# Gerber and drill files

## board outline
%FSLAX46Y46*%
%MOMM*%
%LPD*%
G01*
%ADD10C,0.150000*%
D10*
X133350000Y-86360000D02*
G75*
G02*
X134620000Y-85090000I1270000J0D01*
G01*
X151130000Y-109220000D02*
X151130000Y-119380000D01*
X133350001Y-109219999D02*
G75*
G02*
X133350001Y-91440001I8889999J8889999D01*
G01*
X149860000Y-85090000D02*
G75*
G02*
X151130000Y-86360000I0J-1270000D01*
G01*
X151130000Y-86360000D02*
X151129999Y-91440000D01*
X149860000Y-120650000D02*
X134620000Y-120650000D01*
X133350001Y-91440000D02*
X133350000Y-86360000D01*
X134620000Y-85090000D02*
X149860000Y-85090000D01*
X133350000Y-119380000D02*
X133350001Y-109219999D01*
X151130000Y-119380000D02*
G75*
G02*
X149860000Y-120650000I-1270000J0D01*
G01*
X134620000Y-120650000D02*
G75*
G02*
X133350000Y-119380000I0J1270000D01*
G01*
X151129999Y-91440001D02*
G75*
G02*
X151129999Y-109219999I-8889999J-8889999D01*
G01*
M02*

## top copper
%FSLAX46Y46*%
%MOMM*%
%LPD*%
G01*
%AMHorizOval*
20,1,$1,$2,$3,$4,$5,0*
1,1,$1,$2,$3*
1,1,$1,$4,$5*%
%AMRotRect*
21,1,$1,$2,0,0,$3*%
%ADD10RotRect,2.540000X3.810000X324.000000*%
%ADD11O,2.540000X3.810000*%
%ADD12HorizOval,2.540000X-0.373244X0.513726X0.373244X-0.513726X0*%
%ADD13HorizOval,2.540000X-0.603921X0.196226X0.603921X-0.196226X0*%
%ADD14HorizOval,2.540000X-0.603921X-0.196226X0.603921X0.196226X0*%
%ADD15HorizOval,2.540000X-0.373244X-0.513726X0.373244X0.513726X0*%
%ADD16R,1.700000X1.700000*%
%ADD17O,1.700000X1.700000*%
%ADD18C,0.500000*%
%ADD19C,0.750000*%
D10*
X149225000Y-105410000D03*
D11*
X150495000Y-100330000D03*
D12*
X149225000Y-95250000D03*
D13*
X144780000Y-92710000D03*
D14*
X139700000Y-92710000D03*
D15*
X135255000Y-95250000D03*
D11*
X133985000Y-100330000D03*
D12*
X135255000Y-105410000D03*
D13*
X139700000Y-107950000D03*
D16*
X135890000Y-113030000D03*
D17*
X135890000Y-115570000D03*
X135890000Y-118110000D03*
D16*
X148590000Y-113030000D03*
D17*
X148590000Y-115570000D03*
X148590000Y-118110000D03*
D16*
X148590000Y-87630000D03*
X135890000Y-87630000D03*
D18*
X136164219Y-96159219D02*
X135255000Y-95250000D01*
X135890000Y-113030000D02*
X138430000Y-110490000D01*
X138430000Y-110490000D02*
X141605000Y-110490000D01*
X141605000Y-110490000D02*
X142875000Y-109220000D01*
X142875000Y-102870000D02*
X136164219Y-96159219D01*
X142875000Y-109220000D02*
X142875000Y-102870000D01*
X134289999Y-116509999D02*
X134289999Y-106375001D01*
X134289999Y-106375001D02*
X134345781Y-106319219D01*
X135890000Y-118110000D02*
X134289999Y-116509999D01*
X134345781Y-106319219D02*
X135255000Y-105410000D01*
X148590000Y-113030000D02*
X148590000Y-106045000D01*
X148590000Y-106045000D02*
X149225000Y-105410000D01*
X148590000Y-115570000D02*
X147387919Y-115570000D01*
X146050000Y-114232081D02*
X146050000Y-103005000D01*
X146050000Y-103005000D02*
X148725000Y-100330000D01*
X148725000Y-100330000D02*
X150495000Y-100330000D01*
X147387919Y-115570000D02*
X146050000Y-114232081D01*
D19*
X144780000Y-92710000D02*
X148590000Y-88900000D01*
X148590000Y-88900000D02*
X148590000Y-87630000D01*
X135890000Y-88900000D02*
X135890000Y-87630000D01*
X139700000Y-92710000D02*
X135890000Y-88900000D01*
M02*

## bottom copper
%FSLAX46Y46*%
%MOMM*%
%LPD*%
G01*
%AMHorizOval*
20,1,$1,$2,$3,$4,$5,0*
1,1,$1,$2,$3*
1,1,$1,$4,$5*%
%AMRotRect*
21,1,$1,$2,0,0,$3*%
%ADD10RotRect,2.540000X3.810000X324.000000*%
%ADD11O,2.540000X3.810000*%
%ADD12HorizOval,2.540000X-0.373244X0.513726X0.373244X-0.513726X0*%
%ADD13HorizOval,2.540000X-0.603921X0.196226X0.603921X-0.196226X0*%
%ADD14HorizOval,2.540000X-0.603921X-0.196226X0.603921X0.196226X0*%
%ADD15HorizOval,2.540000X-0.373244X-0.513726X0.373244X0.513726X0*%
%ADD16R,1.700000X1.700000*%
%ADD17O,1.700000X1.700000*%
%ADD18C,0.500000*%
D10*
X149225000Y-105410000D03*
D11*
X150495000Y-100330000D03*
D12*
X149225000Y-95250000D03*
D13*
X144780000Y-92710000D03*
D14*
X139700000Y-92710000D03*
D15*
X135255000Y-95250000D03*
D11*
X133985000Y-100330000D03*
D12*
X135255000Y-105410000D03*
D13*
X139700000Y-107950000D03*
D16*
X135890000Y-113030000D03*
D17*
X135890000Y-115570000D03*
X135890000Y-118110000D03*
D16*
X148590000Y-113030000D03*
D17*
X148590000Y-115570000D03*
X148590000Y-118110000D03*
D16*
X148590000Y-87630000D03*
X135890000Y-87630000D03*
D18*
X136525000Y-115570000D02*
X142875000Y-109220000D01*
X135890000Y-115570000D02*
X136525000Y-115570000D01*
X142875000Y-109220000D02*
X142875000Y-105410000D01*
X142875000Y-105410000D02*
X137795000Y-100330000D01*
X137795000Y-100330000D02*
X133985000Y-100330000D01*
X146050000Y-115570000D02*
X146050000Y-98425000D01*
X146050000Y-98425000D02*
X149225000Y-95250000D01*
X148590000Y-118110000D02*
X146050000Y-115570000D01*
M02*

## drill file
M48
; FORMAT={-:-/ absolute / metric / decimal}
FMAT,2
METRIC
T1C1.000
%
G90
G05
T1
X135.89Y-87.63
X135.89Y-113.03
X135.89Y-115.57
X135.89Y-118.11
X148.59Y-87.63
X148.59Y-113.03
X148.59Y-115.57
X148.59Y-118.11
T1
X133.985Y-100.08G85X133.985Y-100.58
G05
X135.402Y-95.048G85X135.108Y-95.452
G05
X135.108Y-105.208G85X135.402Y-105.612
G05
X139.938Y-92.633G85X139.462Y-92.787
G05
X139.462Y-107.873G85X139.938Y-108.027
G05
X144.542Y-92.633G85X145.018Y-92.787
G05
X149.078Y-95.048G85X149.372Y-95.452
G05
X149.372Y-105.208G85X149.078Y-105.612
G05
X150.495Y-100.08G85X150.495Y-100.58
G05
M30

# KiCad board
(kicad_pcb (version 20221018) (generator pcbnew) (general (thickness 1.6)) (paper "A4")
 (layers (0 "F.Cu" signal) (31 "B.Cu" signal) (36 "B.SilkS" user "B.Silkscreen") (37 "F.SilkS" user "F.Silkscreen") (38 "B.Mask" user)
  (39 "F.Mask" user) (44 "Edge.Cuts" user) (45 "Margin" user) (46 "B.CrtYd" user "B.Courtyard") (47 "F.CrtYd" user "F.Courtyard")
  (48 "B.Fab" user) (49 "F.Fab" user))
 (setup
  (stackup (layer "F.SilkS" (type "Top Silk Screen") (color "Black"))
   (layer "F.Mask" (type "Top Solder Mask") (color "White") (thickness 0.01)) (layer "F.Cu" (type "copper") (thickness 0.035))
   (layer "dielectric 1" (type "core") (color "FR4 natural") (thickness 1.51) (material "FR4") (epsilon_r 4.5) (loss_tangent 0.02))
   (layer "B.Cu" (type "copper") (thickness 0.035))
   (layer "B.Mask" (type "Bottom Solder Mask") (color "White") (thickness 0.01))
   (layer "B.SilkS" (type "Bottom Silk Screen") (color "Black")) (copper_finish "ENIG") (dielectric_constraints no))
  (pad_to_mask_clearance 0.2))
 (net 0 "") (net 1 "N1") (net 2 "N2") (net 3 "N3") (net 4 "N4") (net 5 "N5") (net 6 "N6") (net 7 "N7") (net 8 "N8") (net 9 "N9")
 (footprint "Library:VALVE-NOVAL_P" (layer "F.Cu") (at 149.86 105.41)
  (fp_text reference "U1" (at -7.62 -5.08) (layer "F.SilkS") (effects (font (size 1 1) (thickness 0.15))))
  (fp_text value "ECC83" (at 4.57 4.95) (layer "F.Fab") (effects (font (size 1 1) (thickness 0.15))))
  (pad "1" thru_hole rect (at -0.635 0 324) (size 2.54 3.81) (drill oval 1 1.5) (layers "*.Cu" "*.Mask") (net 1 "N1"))
  (pad "2" thru_hole oval (at 0.635 -5.08) (size 2.54 3.81) (drill oval 1 1.5) (layers "*.Cu" "*.Mask") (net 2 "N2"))
  (pad "3" thru_hole oval (at -0.635 -10.16 36) (size 2.54 3.81) (drill oval 1 1.5) (layers "*.Cu" "*.Mask") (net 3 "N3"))
  (pad "4" thru_hole oval (at -5.08 -12.7 72) (size 2.54 3.81) (drill oval 1 1.5) (layers "*.Cu" "*.Mask") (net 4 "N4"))
  (pad "5" thru_hole oval (at -10.16 -12.7 288) (size 2.54 3.81) (drill oval 1 1.5) (layers "*.Cu" "*.Mask") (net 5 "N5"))
  (pad "6" thru_hole oval (at -14.605 -10.16 324) (size 2.54 3.81) (drill oval 1 1.5) (layers "*.Cu" "*.Mask") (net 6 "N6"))
  (pad "7" thru_hole oval (at -15.875 -5.08) (size 2.54 3.81) (drill oval 1 1.5) (layers "*.Cu" "*.Mask") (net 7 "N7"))
  (pad "8" thru_hole oval (at -14.605 0 36) (size 2.54 3.81) (drill oval 1 1.5) (layers "*.Cu" "*.Mask") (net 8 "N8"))
  (pad "9" thru_hole oval (at -10.16 2.54 72) (size 2.54 3.81) (drill oval 1 1.5) (layers "*.Cu" "*.Mask") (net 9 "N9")))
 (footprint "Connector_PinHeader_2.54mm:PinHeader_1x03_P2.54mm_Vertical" (layer "B.Cu") (at 135.89 113.03 180)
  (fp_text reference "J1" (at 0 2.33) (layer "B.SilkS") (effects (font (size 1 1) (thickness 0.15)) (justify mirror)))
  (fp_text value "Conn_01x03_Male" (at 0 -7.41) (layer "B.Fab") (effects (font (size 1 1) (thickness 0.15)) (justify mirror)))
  (pad "1" thru_hole rect (at 0 0 180) (size 1.7 1.7) (drill 1) (layers "*.Cu" "*.Mask") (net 6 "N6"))
  (pad "2" thru_hole oval (at 0 -2.54 180) (size 1.7 1.7) (drill 1) (layers "*.Cu" "*.Mask") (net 7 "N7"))
  (pad "3" thru_hole oval (at 0 -5.08 180) (size 1.7 1.7) (drill 1) (layers "*.Cu" "*.Mask") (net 8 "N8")))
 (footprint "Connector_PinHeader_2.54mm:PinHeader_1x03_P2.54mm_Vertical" (layer "B.Cu") (at 148.59 113.03 180)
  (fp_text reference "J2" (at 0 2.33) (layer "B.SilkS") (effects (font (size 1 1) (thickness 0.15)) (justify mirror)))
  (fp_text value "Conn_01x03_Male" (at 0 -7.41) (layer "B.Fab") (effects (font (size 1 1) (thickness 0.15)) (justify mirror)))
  (pad "1" thru_hole rect (at 0 0 180) (size 1.7 1.7) (drill 1) (layers "*.Cu" "*.Mask") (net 1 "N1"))
  (pad "2" thru_hole oval (at 0 -2.54 180) (size 1.7 1.7) (drill 1) (layers "*.Cu" "*.Mask") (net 2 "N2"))
  (pad "3" thru_hole oval (at 0 -5.08 180) (size 1.7 1.7) (drill 1) (layers "*.Cu" "*.Mask") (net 3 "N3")))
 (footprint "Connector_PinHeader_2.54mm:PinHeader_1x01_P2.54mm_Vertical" (layer "B.Cu") (at 148.59 87.63)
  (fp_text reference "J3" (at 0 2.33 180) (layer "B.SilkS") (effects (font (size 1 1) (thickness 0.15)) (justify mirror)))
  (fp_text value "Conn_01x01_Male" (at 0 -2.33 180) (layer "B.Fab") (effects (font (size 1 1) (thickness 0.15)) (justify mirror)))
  (pad "1" thru_hole rect (at 0 0) (size 1.7 1.7) (drill 1) (layers "*.Cu" "*.Mask") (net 4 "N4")))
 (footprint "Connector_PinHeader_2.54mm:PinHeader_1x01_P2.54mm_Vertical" (layer "B.Cu") (at 135.89 87.63)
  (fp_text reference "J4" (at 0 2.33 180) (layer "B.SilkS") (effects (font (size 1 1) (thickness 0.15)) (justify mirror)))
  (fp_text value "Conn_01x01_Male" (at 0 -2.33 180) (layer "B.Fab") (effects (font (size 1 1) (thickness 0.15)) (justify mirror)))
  (pad "1" thru_hole rect (at 0 0) (size 1.7 1.7) (drill 1) (layers "*.Cu" "*.Mask") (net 5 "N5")))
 (gr_arc (start 133.35 86.36) (mid 133.721974 85.461974) (end 134.62 85.09) (stroke (width 0.15) (type solid)) (layer "Edge.Cuts"))
 (gr_line (start 151.13 109.22) (end 151.13 119.38) (stroke (width 0.15) (type solid)) (layer "Edge.Cuts"))
 (gr_arc (start 133.350001 109.219999) (mid 129.667643 100.33) (end 133.350001 91.440001) (stroke (width 0.15) (type solid))
  (layer "Edge.Cuts"))
 (gr_arc (start 149.86 85.09) (mid 150.758026 85.461974) (end 151.13 86.36) (stroke (width 0.15) (type solid)) (layer "Edge.Cuts"))
 (gr_line (start 151.13 86.36) (end 151.129999 91.44) (stroke (width 0.15) (type solid)) (layer "Edge.Cuts"))
 (gr_line (start 149.86 120.65) (end 134.62 120.65) (stroke (width 0.15) (type solid)) (layer "Edge.Cuts"))
 (gr_line (start 133.350001 91.44) (end 133.35 86.36) (stroke (width 0.15) (type solid)) (layer "Edge.Cuts"))
 (gr_line (start 134.62 85.09) (end 149.86 85.09) (stroke (width 0.15) (type solid)) (layer "Edge.Cuts"))
 (gr_line (start 133.35 119.38) (end 133.350001 109.219999) (stroke (width 0.15) (type solid)) (layer "Edge.Cuts"))
 (gr_arc (start 151.13 119.38) (mid 150.758026 120.278026) (end 149.86 120.65) (stroke (width 0.15) (type solid)) (layer "Edge.Cuts"))
 (gr_arc (start 134.62 120.65) (mid 133.721974 120.278026) (end 133.35 119.38) (stroke (width 0.15) (type solid)) (layer "Edge.Cuts"))
 (gr_arc (start 151.129999 91.440001) (mid 154.812357 100.33) (end 151.129999 109.219999) (stroke (width 0.15) (type solid))
  (layer "Edge.Cuts"))
 (segment (start 136.164219 96.159219) (end 135.255 95.25) (width 0.5) (layer "F.Cu") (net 6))
 (segment (start 135.89 113.03) (end 138.43 110.49) (width 0.5) (layer "F.Cu") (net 6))
 (segment (start 138.43 110.49) (end 141.605 110.49) (width 0.5) (layer "F.Cu") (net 6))
 (segment (start 141.605 110.49) (end 142.875 109.22) (width 0.5) (layer "F.Cu") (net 6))
 (segment (start 142.875 102.87) (end 136.164219 96.159219) (width 0.5) (layer "F.Cu") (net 6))
 (segment (start 142.875 109.22) (end 142.875 102.87) (width 0.5) (layer "F.Cu") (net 6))
 (segment (start 136.525 115.57) (end 142.875 109.22) (width 0.5) (layer "B.Cu") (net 7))
 (segment (start 135.89 115.57) (end 136.525 115.57) (width 0.5) (layer "B.Cu") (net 7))
 (segment (start 142.875 109.22) (end 142.875 105.41) (width 0.5) (layer "B.Cu") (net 7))
 (segment (start 142.875 105.41) (end 137.795 100.33) (width 0.5) (layer "B.Cu") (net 7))
 (segment (start 137.795 100.33) (end 133.985 100.33) (width 0.5) (layer "B.Cu") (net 7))
 (segment (start 134.289999 116.509999) (end 134.289999 106.375001) (width 0.5) (layer "F.Cu") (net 8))
 (segment (start 134.289999 106.375001) (end 134.345781 106.319219) (width 0.5) (layer "F.Cu") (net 8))
 (segment (start 135.89 118.11) (end 134.289999 116.509999) (width 0.5) (layer "F.Cu") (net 8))
 (segment (start 134.345781 106.319219) (end 135.255 105.41) (width 0.5) (layer "F.Cu") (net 8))
 (segment (start 148.59 113.03) (end 148.59 106.045) (width 0.5) (layer "F.Cu") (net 1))
 (segment (start 148.59 106.045) (end 149.225 105.41) (width 0.5) (layer "F.Cu") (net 1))
 (segment (start 148.59 115.57) (end 147.387919 115.57) (width 0.5) (layer "F.Cu") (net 2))
 (segment (start 146.05 114.232081) (end 146.05 103.005) (width 0.5) (layer "F.Cu") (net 2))
 (segment (start 146.05 103.005) (end 148.725 100.33) (width 0.5) (layer "F.Cu") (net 2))
 (segment (start 148.725 100.33) (end 150.495 100.33) (width 0.5) (layer "F.Cu") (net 2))
 (segment (start 147.387919 115.57) (end 146.05 114.232081) (width 0.5) (layer "F.Cu") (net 2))
 (segment (start 146.05 115.57) (end 146.05 98.425) (width 0.5) (layer "B.Cu") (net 3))
 (segment (start 146.05 98.425) (end 149.225 95.25) (width 0.5) (layer "B.Cu") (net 3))
 (segment (start 148.59 118.11) (end 146.05 115.57) (width 0.5) (layer "B.Cu") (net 3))
 (segment (start 144.78 92.71) (end 148.59 88.9) (width 0.75) (layer "F.Cu") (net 4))
 (segment (start 148.59 88.9) (end 148.59 87.63) (width 0.75) (layer "F.Cu") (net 4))
 (segment (start 135.89 88.9) (end 135.89 87.63) (width 0.75) (layer "F.Cu") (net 5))
 (segment (start 139.7 92.71) (end 135.89 88.9) (width 0.75) (layer "F.Cu") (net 5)))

